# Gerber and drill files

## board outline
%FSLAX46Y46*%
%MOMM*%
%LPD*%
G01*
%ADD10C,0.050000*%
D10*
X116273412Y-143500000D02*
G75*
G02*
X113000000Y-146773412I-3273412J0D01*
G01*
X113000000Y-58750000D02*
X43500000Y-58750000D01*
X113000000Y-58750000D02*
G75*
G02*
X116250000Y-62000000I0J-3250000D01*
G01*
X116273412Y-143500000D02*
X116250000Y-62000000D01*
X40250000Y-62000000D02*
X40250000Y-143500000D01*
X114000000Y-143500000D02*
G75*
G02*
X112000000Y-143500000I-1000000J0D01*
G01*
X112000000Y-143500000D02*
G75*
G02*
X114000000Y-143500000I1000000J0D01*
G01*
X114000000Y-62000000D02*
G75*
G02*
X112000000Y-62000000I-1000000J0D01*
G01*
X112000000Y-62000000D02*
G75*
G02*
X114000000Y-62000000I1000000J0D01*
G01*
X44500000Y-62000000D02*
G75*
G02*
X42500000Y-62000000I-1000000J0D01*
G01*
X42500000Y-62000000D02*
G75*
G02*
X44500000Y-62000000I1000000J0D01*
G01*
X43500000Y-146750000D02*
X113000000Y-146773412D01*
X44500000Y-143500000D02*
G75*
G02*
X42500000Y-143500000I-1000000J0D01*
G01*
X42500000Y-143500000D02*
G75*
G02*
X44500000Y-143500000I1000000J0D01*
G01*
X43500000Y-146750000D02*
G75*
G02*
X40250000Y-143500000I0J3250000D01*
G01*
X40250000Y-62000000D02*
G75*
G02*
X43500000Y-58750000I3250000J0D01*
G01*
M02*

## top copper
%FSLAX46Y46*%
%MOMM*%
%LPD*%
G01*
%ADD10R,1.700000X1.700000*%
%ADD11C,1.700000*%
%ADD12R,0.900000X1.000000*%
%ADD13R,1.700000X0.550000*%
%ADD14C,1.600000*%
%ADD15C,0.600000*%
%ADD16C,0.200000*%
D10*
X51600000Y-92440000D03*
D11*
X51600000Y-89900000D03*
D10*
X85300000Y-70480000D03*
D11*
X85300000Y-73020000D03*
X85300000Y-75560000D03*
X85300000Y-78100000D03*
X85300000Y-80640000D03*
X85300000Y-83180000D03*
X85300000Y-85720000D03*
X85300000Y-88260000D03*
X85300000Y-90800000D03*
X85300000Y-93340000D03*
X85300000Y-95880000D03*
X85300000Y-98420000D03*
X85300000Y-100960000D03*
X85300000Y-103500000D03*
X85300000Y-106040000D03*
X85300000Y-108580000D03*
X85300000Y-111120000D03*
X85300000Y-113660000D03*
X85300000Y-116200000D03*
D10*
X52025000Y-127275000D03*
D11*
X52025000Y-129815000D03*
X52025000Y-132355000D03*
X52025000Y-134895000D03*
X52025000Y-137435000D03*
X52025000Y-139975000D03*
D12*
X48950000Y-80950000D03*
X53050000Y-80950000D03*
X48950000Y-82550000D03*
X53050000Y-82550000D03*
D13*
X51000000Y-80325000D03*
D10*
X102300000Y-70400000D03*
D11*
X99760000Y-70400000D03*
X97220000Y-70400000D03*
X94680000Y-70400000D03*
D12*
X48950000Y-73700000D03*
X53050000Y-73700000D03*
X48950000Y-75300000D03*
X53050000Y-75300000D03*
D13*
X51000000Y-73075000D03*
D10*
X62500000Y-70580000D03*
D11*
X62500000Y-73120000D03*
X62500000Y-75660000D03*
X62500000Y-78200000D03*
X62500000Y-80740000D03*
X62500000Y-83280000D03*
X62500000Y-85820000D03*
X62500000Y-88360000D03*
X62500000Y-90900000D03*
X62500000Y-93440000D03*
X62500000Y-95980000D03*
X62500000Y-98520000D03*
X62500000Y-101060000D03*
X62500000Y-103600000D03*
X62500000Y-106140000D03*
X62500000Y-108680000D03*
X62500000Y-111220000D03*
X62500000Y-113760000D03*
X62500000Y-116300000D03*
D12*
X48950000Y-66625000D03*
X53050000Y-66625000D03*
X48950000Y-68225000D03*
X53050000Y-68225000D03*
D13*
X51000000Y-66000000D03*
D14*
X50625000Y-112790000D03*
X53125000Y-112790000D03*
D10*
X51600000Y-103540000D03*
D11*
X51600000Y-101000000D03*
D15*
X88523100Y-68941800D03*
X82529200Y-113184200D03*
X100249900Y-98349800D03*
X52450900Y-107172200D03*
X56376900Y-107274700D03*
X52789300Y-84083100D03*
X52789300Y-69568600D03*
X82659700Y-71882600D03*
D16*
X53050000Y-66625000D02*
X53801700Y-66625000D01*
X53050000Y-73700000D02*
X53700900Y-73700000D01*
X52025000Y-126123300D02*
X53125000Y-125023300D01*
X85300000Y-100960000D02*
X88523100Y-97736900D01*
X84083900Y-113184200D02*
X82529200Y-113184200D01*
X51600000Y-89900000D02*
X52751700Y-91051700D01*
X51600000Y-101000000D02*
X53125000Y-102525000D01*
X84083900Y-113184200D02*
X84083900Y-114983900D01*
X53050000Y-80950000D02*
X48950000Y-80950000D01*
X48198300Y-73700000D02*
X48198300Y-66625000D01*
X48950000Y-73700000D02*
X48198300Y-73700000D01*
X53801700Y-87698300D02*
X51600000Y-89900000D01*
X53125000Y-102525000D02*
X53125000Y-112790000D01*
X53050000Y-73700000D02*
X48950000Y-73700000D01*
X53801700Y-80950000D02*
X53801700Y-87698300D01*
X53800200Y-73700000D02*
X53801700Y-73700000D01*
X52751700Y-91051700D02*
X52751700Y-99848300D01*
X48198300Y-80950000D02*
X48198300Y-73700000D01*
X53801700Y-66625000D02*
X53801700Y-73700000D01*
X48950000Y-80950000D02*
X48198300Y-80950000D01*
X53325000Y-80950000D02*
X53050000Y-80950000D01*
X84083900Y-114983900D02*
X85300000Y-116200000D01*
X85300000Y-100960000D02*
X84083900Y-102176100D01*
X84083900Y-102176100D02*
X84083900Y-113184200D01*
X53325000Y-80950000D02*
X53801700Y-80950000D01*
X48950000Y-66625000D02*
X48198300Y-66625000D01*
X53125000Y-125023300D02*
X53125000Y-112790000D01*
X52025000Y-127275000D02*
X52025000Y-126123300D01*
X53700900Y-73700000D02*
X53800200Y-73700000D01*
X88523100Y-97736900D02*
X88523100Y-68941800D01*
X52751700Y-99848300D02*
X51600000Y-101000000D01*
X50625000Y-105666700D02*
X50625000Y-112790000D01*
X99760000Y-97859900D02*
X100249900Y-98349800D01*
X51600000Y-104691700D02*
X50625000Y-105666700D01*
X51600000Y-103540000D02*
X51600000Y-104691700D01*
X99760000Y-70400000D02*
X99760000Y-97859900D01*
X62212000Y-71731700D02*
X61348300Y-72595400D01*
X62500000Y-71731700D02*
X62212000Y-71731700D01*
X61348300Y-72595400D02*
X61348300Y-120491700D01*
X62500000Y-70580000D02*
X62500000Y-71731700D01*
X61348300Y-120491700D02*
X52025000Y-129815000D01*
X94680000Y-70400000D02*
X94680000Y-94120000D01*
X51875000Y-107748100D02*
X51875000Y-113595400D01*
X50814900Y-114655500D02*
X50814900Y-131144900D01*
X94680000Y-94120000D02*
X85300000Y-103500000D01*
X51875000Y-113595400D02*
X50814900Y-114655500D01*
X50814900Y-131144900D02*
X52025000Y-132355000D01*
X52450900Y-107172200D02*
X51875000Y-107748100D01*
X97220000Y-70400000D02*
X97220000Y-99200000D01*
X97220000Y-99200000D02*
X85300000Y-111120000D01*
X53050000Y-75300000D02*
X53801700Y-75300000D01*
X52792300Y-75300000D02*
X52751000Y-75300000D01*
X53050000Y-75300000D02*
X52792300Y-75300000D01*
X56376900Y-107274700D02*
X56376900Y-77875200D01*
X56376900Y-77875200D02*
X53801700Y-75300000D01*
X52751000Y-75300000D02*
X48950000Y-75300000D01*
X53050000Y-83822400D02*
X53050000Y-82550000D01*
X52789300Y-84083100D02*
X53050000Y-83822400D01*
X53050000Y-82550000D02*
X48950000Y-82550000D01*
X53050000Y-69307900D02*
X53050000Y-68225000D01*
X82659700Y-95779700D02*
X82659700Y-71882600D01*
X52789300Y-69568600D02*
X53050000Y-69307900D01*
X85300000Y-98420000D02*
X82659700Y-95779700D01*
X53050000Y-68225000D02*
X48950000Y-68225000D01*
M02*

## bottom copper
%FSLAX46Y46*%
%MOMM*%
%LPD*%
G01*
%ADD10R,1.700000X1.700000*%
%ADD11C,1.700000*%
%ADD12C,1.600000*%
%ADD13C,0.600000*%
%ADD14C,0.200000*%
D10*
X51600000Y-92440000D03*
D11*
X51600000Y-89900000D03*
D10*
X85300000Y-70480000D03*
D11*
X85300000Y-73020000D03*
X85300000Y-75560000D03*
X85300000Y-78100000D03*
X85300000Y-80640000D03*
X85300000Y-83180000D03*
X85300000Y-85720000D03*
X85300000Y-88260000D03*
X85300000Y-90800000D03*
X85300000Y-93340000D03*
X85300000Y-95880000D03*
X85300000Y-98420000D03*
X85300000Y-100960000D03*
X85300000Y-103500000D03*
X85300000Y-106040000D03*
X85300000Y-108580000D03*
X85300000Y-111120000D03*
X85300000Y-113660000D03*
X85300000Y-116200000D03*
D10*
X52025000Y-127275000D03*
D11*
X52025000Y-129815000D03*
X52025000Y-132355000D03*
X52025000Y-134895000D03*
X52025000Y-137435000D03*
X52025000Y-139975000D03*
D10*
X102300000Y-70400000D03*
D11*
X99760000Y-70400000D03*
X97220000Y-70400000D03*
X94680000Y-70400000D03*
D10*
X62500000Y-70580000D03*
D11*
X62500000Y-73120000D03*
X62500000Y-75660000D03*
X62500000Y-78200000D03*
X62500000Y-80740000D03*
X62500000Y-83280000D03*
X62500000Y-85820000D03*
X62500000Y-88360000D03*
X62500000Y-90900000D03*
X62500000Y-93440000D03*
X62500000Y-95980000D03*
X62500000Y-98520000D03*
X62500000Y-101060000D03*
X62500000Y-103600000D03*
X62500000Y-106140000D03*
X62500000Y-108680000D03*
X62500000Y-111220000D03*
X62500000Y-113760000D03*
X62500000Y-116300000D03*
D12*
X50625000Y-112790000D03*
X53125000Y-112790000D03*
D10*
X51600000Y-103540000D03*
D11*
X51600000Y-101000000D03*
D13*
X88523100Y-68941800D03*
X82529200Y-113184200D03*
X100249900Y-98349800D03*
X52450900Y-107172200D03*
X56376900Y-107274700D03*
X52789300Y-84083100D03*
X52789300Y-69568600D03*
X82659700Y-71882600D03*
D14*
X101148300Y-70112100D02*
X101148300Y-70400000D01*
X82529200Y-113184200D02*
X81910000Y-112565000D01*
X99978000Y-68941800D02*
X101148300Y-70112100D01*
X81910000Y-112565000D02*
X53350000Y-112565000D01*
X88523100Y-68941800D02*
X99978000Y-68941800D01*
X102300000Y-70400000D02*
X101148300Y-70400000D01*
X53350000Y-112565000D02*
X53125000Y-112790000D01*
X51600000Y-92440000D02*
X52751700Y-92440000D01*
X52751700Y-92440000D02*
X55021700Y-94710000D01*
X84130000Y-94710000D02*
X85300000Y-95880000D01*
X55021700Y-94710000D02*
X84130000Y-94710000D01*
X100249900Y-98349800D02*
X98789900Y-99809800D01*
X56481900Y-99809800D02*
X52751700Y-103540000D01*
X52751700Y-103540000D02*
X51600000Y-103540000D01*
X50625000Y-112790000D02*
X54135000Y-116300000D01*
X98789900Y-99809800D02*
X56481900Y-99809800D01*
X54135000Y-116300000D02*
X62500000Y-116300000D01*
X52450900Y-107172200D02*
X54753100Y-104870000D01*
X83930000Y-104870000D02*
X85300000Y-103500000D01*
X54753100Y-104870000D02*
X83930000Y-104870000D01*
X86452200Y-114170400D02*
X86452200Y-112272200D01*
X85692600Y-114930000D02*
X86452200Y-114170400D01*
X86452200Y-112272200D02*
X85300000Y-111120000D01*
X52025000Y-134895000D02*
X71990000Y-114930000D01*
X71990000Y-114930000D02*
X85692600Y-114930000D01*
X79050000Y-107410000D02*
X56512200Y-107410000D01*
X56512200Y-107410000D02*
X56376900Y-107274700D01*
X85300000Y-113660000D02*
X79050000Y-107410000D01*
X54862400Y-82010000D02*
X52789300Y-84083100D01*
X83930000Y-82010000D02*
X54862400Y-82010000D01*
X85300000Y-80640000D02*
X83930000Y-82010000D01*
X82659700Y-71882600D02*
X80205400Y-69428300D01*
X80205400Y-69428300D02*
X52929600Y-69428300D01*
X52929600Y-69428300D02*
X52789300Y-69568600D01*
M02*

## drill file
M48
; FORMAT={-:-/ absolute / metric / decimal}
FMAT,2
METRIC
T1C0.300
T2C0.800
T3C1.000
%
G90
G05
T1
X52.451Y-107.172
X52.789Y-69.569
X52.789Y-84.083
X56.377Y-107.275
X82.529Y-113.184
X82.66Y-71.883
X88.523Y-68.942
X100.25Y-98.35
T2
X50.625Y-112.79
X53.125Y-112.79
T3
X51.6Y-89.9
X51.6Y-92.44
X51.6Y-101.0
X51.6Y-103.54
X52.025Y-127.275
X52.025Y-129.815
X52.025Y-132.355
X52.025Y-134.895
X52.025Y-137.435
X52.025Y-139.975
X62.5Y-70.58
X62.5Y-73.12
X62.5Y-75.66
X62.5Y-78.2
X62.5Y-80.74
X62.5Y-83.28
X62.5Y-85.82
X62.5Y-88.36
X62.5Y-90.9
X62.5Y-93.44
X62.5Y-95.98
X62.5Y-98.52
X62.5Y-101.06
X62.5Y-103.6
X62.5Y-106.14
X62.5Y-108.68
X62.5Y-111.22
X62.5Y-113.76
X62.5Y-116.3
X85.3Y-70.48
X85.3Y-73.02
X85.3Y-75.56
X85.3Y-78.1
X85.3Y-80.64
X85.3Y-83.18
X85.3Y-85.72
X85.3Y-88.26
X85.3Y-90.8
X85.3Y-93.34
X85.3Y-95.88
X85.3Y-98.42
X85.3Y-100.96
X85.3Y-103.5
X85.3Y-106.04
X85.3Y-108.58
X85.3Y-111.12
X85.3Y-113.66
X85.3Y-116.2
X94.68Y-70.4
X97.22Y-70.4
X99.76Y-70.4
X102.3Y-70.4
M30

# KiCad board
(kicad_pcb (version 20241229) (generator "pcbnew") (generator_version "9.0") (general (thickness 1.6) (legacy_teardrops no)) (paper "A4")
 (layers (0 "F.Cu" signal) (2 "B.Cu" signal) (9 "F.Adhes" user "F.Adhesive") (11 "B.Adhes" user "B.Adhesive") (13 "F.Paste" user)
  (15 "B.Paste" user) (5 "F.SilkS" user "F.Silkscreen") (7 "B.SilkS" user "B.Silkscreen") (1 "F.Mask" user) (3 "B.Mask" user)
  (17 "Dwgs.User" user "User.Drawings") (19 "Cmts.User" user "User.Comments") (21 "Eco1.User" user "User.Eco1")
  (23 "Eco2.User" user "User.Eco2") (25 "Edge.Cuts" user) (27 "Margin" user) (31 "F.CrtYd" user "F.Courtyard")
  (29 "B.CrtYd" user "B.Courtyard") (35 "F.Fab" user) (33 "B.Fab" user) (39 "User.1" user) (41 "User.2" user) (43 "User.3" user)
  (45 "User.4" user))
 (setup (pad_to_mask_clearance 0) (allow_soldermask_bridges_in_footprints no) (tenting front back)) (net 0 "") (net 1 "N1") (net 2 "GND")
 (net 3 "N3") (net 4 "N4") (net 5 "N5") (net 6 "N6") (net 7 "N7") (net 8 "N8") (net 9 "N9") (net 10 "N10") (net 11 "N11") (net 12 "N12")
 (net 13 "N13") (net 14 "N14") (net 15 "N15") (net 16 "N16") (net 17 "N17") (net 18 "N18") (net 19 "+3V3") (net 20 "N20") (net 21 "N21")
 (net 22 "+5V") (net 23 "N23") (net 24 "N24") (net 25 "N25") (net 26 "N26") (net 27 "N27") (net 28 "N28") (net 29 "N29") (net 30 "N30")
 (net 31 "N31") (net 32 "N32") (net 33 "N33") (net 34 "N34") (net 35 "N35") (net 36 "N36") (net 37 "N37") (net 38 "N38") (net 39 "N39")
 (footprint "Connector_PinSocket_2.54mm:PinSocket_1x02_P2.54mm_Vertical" (layer "F.Cu") (at 51.6 92.44 180)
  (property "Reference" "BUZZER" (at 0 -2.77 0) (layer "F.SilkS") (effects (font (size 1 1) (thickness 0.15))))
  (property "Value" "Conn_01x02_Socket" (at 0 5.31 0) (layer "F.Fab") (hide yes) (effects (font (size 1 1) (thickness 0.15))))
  (pad "1" thru_hole rect (at 0 0 180) (size 1.7 1.7) (drill 1) (layers "*.Cu" "*.Mask") (remove_unused_layers no) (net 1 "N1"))
  (pad "2" thru_hole circle (at 0 2.54 180) (size 1.7 1.7) (drill 1) (layers "*.Cu" "*.Mask") (remove_unused_layers no) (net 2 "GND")))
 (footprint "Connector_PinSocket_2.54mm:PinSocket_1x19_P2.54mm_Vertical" (layer "F.Cu") (at 85.3 70.48)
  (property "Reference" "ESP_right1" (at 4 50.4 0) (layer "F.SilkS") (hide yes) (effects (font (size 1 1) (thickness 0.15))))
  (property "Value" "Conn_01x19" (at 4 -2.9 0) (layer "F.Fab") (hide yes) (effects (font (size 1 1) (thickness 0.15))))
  (pad "1" thru_hole rect (at 0 0) (size 1.7 1.7) (drill 1) (layers "*.Cu" "*.Mask") (remove_unused_layers no) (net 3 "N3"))
  (pad "2" thru_hole circle (at 0 2.54) (size 1.7 1.7) (drill 1) (layers "*.Cu" "*.Mask") (remove_unused_layers no) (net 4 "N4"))
  (pad "3" thru_hole circle (at 0 5.08) (size 1.7 1.7) (drill 1) (layers "*.Cu" "*.Mask") (remove_unused_layers no) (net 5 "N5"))
  (pad "4" thru_hole circle (at 0 7.62) (size 1.7 1.7) (drill 1) (layers "*.Cu" "*.Mask") (remove_unused_layers no) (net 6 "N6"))
  (pad "5" thru_hole circle (at 0 10.16) (size 1.7 1.7) (drill 1) (layers "*.Cu" "*.Mask") (remove_unused_layers no) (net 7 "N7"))
  (pad "6" thru_hole circle (at 0 12.7) (size 1.7 1.7) (drill 1) (layers "*.Cu" "*.Mask") (remove_unused_layers no) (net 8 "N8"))
  (pad "7" thru_hole circle (at 0 15.24) (size 1.7 1.7) (drill 1) (layers "*.Cu" "*.Mask") (remove_unused_layers no) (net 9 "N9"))
  (pad "8" thru_hole circle (at 0 17.78) (size 1.7 1.7) (drill 1) (layers "*.Cu" "*.Mask") (remove_unused_layers no) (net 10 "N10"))
  (pad "9" thru_hole circle (at 0 20.32) (size 1.7 1.7) (drill 1) (layers "*.Cu" "*.Mask") (remove_unused_layers no) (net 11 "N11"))
  (pad "10" thru_hole circle (at 0 22.86) (size 1.7 1.7) (drill 1) (layers "*.Cu" "*.Mask") (remove_unused_layers no) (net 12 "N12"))
  (pad "11" thru_hole circle (at 0 25.4) (size 1.7 1.7) (drill 1) (layers "*.Cu" "*.Mask") (remove_unused_layers no) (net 1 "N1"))
  (pad "12" thru_hole circle (at 0 27.94) (size 1.7 1.7) (drill 1) (layers "*.Cu" "*.Mask") (remove_unused_layers no) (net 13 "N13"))
  (pad "13" thru_hole circle (at 0 30.48) (size 1.7 1.7) (drill 1) (layers "*.Cu" "*.Mask") (remove_unused_layers no) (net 2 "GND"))
  (pad "14" thru_hole circle (at 0 33.02) (size 1.7 1.7) (drill 1) (layers "*.Cu" "*.Mask") (remove_unused_layers no) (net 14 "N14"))
  (pad "15" thru_hole circle (at 0 35.56) (size 1.7 1.7) (drill 1) (layers "*.Cu" "*.Mask") (remove_unused_layers no) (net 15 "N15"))
  (pad "16" thru_hole circle (at 0 38.1) (size 1.7 1.7) (drill 1) (layers "*.Cu" "*.Mask") (remove_unused_layers no) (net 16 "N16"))
  (pad "17" thru_hole circle (at 0 40.64) (size 1.7 1.7) (drill 1) (layers "*.Cu" "*.Mask") (remove_unused_layers no) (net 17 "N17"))
  (pad "18" thru_hole circle (at 0 43.18) (size 1.7 1.7) (drill 1) (layers "*.Cu" "*.Mask") (remove_unused_layers no) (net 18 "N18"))
  (pad "19" thru_hole circle (at 0 45.72) (size 1.7 1.7) (drill 1) (layers "*.Cu" "*.Mask") (remove_unused_layers no) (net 2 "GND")))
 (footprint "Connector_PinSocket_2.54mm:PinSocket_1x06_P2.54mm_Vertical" (layer "F.Cu") (at 52.025 127.275)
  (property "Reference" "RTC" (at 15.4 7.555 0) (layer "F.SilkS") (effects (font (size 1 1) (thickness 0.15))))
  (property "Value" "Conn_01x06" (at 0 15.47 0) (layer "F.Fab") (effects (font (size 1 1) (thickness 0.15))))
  (pad "1" thru_hole rect (at 0 0) (size 1.7 1.7) (drill 1) (layers "*.Cu" "*.Mask") (remove_unused_layers no) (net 2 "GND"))
  (pad "2" thru_hole circle (at 0 2.54) (size 1.7 1.7) (drill 1) (layers "*.Cu" "*.Mask") (remove_unused_layers no) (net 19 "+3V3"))
  (pad "3" thru_hole circle (at 0 5.08) (size 1.7 1.7) (drill 1) (layers "*.Cu" "*.Mask") (remove_unused_layers no) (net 14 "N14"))
  (pad "4" thru_hole circle (at 0 7.62) (size 1.7 1.7) (drill 1) (layers "*.Cu" "*.Mask") (remove_unused_layers no) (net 17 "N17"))
  (pad "5" thru_hole circle (at 0 10.16) (size 1.7 1.7) (drill 1) (layers "*.Cu" "*.Mask") (remove_unused_layers no) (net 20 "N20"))
  (pad "6" thru_hole circle (at 0 12.7) (size 1.7 1.7) (drill 1) (layers "*.Cu" "*.Mask") (remove_unused_layers no) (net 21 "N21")))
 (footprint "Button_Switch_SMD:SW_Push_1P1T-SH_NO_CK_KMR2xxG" (layer "F.Cu") (at 51 81.75)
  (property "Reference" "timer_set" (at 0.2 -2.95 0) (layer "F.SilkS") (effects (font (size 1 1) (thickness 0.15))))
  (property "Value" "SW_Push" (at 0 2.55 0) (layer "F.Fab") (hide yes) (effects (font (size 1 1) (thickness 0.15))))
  (pad "1" smd rect (at -2.05 -0.8) (size 0.9 1) (layers "F.Cu" "F.Mask" "F.Paste") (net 2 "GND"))
  (pad "1" smd rect (at 2.05 -0.8) (size 0.9 1) (layers "F.Cu" "F.Mask" "F.Paste") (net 2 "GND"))
  (pad "2" smd rect (at -2.05 0.8) (size 0.9 1) (layers "F.Cu" "F.Mask" "F.Paste") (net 7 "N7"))
  (pad "2" smd rect (at 2.05 0.8) (size 0.9 1) (layers "F.Cu" "F.Mask" "F.Paste") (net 7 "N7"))
  (pad "SH" smd rect (at 0 -1.425) (size 1.7 0.55) (layers "F.Cu" "F.Mask" "F.Paste")))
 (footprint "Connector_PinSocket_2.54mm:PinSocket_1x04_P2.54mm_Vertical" (layer "F.Cu") (at 102.3 70.4 -90)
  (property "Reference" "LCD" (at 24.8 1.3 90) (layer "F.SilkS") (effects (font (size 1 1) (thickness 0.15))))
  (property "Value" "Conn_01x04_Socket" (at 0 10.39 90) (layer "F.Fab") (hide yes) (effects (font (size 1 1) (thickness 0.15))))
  (pad "1" thru_hole rect (at 0 0 270) (size 1.7 1.7) (drill 1) (layers "*.Cu" "*.Mask") (remove_unused_layers no) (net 2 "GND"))
  (pad "2" thru_hole circle (at 0 2.54 270) (size 1.7 1.7) (drill 1) (layers "*.Cu" "*.Mask") (remove_unused_layers no) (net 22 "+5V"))
  (pad "3" thru_hole circle (at 0 5.08 270) (size 1.7 1.7) (drill 1) (layers "*.Cu" "*.Mask") (remove_unused_layers no) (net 17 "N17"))
  (pad "4" thru_hole circle (at 0 7.62 270) (size 1.7 1.7) (drill 1) (layers "*.Cu" "*.Mask") (remove_unused_layers no) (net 14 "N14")))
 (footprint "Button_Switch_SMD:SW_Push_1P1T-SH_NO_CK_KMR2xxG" (layer "F.Cu") (at 51 74.5)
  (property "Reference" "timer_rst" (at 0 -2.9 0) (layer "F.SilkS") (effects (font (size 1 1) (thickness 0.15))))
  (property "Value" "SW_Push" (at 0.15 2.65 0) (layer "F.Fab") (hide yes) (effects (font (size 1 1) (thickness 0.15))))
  (pad "1" smd rect (at -2.05 -0.8) (size 0.9 1) (layers "F.Cu" "F.Mask" "F.Paste") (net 2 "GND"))
  (pad "1" smd rect (at 2.05 -0.8) (size 0.9 1) (layers "F.Cu" "F.Mask" "F.Paste") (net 2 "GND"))
  (pad "2" smd rect (at -2.05 0.8) (size 0.9 1) (layers "F.Cu" "F.Mask" "F.Paste") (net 18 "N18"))
  (pad "2" smd rect (at 2.05 0.8) (size 0.9 1) (layers "F.Cu" "F.Mask" "F.Paste") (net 18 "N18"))
  (pad "SH" smd rect (at 0 -1.425) (size 1.7 0.55) (layers "F.Cu" "F.Mask" "F.Paste")))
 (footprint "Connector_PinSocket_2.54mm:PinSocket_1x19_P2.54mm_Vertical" (layer "F.Cu") (at 62.5 70.58)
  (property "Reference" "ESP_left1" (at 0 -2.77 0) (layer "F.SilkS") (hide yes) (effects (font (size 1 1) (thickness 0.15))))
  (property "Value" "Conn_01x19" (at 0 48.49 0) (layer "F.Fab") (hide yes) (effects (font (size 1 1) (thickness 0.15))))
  (pad "1" thru_hole rect (at 0 0) (size 1.7 1.7) (drill 1) (layers "*.Cu" "*.Mask") (remove_unused_layers no) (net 19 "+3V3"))
  (pad "2" thru_hole circle (at 0 2.54) (size 1.7 1.7) (drill 1) (layers "*.Cu" "*.Mask") (remove_unused_layers no) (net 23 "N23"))
  (pad "3" thru_hole circle (at 0 5.08) (size 1.7 1.7) (drill 1) (layers "*.Cu" "*.Mask") (remove_unused_layers no) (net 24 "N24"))
  (pad "4" thru_hole circle (at 0 7.62) (size 1.7 1.7) (drill 1) (layers "*.Cu" "*.Mask") (remove_unused_layers no) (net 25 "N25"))
  (pad "5" thru_hole circle (at 0 10.16) (size 1.7 1.7) (drill 1) (layers "*.Cu" "*.Mask") (remove_unused_layers no) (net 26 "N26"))
  (pad "6" thru_hole circle (at 0 12.7) (size 1.7 1.7) (drill 1) (layers "*.Cu" "*.Mask") (remove_unused_layers no) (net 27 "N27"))
  (pad "7" thru_hole circle (at 0 15.24) (size 1.7 1.7) (drill 1) (layers "*.Cu" "*.Mask") (remove_unused_layers no) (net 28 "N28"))
  (pad "8" thru_hole circle (at 0 17.78) (size 1.7 1.7) (drill 1) (layers "*.Cu" "*.Mask") (remove_unused_layers no) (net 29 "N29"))
  (pad "9" thru_hole circle (at 0 20.32) (size 1.7 1.7) (drill 1) (layers "*.Cu" "*.Mask") (remove_unused_layers no) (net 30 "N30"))
  (pad "10" thru_hole circle (at 0 22.86) (size 1.7 1.7) (drill 1) (layers "*.Cu" "*.Mask") (remove_unused_layers no) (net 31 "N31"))
  (pad "11" thru_hole circle (at 0 25.4) (size 1.7 1.7) (drill 1) (layers "*.Cu" "*.Mask") (remove_unused_layers no) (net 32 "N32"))
  (pad "12" thru_hole circle (at 0 27.94) (size 1.7 1.7) (drill 1) (layers "*.Cu" "*.Mask") (remove_unused_layers no) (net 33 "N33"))
  (pad "13" thru_hole circle (at 0 30.48) (size 1.7 1.7) (drill 1) (layers "*.Cu" "*.Mask") (remove_unused_layers no) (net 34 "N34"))
  (pad "14" thru_hole circle (at 0 33.02) (size 1.7 1.7) (drill 1) (layers "*.Cu" "*.Mask") (remove_unused_layers no) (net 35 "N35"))
  (pad "15" thru_hole circle (at 0 35.56) (size 1.7 1.7) (drill 1) (layers "*.Cu" "*.Mask") (remove_unused_layers no) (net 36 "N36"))
  (pad "16" thru_hole circle (at 0 38.1) (size 1.7 1.7) (drill 1) (layers "*.Cu" "*.Mask") (remove_unused_layers no) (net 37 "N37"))
  (pad "17" thru_hole circle (at 0 40.64) (size 1.7 1.7) (drill 1) (layers "*.Cu" "*.Mask") (remove_unused_layers no) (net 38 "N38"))
  (pad "18" thru_hole circle (at 0 43.18) (size 1.7 1.7) (drill 1) (layers "*.Cu" "*.Mask") (remove_unused_layers no) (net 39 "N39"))
  (pad "19" thru_hole circle (at 0 45.72) (size 1.7 1.7) (drill 1) (layers "*.Cu" "*.Mask") (remove_unused_layers no) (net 22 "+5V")))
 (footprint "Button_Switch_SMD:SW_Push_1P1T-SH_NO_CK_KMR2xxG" (layer "F.Cu") (at 51 67.425)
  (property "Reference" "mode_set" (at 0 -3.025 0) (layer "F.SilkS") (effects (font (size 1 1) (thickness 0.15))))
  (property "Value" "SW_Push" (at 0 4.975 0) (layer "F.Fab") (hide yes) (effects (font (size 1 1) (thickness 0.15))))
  (pad "1" smd rect (at -2.05 -0.8) (size 0.9 1) (layers "F.Cu" "F.Mask" "F.Paste") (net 2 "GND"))
  (pad "1" smd rect (at 2.05 -0.8) (size 0.9 1) (layers "F.Cu" "F.Mask" "F.Paste") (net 2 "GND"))
  (pad "2" smd rect (at -2.05 0.8) (size 0.9 1) (layers "F.Cu" "F.Mask" "F.Paste") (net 13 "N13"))
  (pad "2" smd rect (at 2.05 0.8) (size 0.9 1) (layers "F.Cu" "F.Mask" "F.Paste") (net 13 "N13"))
  (pad "SH" smd rect (at 0 -1.425) (size 1.7 0.55) (layers "F.Cu" "F.Mask" "F.Paste")))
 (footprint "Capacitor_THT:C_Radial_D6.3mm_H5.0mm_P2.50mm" (layer "F.Cu") (at 50.625 112.79)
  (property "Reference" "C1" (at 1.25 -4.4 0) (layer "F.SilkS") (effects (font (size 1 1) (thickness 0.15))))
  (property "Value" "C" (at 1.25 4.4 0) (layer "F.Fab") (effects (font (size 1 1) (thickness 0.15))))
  (pad "1" thru_hole circle (at 0 0) (size 1.6 1.6) (drill 0.8) (layers "*.Cu" "*.Mask") (remove_unused_layers no) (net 22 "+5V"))
  (pad "2" thru_hole circle (at 2.5 0) (size 1.6 1.6) (drill 0.8) (layers "*.Cu" "*.Mask") (remove_unused_layers no) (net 2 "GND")))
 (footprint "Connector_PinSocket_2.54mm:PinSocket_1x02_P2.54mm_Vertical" (layer "F.Cu") (at 51.6 103.54 180)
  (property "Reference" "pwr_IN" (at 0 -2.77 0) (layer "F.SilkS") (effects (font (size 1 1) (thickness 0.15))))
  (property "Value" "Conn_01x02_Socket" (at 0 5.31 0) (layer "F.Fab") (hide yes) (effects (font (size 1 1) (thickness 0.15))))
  (pad "1" thru_hole rect (at 0 0 180) (size 1.7 1.7) (drill 1) (layers "*.Cu" "*.Mask") (remove_unused_layers no) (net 22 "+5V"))
  (pad "2" thru_hole circle (at 0 2.54 180) (size 1.7 1.7) (drill 1) (layers "*.Cu" "*.Mask") (remove_unused_layers no) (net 2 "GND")))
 (gr_arc (start 116.273412 143.5) (mid 115.314652 145.814652) (end 113 146.773412) (stroke (width 0.05) (type default)) (layer "Edge.Cuts"))
 (gr_line (start 113 58.75) (end 43.5 58.75) (stroke (width 0.05) (type default)) (layer "Edge.Cuts"))
 (gr_arc (start 113 58.75) (mid 115.298097 59.701903) (end 116.25 62) (stroke (width 0.05) (type default)) (layer "Edge.Cuts"))
 (gr_line (start 116.273412 143.5) (end 116.25 62) (stroke (width 0.05) (type default)) (layer "Edge.Cuts"))
 (gr_line (start 40.25 62) (end 40.25 143.5) (stroke (width 0.05) (type default)) (layer "Edge.Cuts"))
 (gr_circle (center 113 143.5) (end 114 143.5) (stroke (width 0.05) (type default)) (fill no) (layer "Edge.Cuts"))
 (gr_circle (center 113 62) (end 114 62) (stroke (width 0.05) (type default)) (fill no) (layer "Edge.Cuts"))
 (gr_circle (center 43.5 62) (end 42.5 62) (stroke (width 0.05) (type default)) (fill no) (layer "Edge.Cuts"))
 (gr_line (start 43.5 146.75) (end 113 146.773412) (stroke (width 0.05) (type default)) (layer "Edge.Cuts"))
 (gr_circle (center 43.5 143.5) (end 42.5 143.5) (stroke (width 0.05) (type default)) (fill no) (layer "Edge.Cuts"))
 (gr_arc (start 43.5 146.75) (mid 41.201903 145.798097) (end 40.25 143.5) (stroke (width 0.05) (type default)) (layer "Edge.Cuts"))
 (gr_arc (start 40.25 62) (mid 41.201903 59.701903) (end 43.5 58.75) (stroke (width 0.05) (type default)) (layer "Edge.Cuts"))
 (segment (start 53.05 66.625) (end 53.8017 66.625) (width 0.2) (layer "F.Cu") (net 2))
 (segment (start 53.05 73.7) (end 53.7009 73.7) (width 0.2) (layer "F.Cu") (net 2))
 (segment (start 52.025 126.1233) (end 53.125 125.0233) (width 0.2) (layer "F.Cu") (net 2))
 (segment (start 85.3 100.96) (end 88.5231 97.7369) (width 0.2) (layer "F.Cu") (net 2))
 (segment (start 84.0839 113.1842) (end 82.5292 113.1842) (width 0.2) (layer "F.Cu") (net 2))
 (segment (start 51.6 89.9) (end 52.7517 91.0517) (width 0.2) (layer "F.Cu") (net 2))
 (segment (start 51.6 101) (end 53.125 102.525) (width 0.2) (layer "F.Cu") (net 2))
 (segment (start 84.0839 113.1842) (end 84.0839 114.9839) (width 0.2) (layer "F.Cu") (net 2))
 (segment (start 53.05 80.95) (end 48.95 80.95) (width 0.2) (layer "F.Cu") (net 2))
 (segment (start 48.1983 73.7) (end 48.1983 66.625) (width 0.2) (layer "F.Cu") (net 2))
 (segment (start 48.95 73.7) (end 48.1983 73.7) (width 0.2) (layer "F.Cu") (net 2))
 (segment (start 53.8017 87.6983) (end 51.6 89.9) (width 0.2) (layer "F.Cu") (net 2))
 (segment (start 53.125 102.525) (end 53.125 112.79) (width 0.2) (layer "F.Cu") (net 2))
 (segment (start 53.05 73.7) (end 48.95 73.7) (width 0.2) (layer "F.Cu") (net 2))
 (segment (start 53.8017 80.95) (end 53.8017 87.6983) (width 0.2) (layer "F.Cu") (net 2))
 (segment (start 53.8002 73.7) (end 53.8017 73.7) (width 0.2) (layer "F.Cu") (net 2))
 (segment (start 52.7517 91.0517) (end 52.7517 99.8483) (width 0.2) (layer "F.Cu") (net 2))
 (segment (start 48.1983 80.95) (end 48.1983 73.7) (width 0.2) (layer "F.Cu") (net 2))
 (segment (start 53.8017 66.625) (end 53.8017 73.7) (width 0.2) (layer "F.Cu") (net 2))
 (segment (start 48.95 80.95) (end 48.1983 80.95) (width 0.2) (layer "F.Cu") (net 2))
 (segment (start 53.325 80.95) (end 53.05 80.95) (width 0.2) (layer "F.Cu") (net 2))
 (segment (start 84.0839 114.9839) (end 85.3 116.2) (width 0.2) (layer "F.Cu") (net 2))
 (segment (start 85.3 100.96) (end 84.0839 102.1761) (width 0.2) (layer "F.Cu") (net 2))
 (segment (start 84.0839 102.1761) (end 84.0839 113.1842) (width 0.2) (layer "F.Cu") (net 2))
 (segment (start 53.325 80.95) (end 53.8017 80.95) (width 0.2) (layer "F.Cu") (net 2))
 (segment (start 48.95 66.625) (end 48.1983 66.625) (width 0.2) (layer "F.Cu") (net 2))
 (segment (start 53.125 125.0233) (end 53.125 112.79) (width 0.2) (layer "F.Cu") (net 2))
 (segment (start 52.025 127.275) (end 52.025 126.1233) (width 0.2) (layer "F.Cu") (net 2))
 (segment (start 53.7009 73.7) (end 53.8002 73.7) (width 0.2) (layer "F.Cu") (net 2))
 (segment (start 88.5231 97.7369) (end 88.5231 68.9418) (width 0.2) (layer "F.Cu") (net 2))
 (segment (start 52.7517 99.8483) (end 51.6 101) (width 0.2) (layer "F.Cu") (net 2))
 (via (at 88.5231 68.9418) (size 0.6) (drill 0.3) (layers "F.Cu" "B.Cu") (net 2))
 (via (at 82.5292 113.1842) (size 0.6) (drill 0.3) (layers "F.Cu" "B.Cu") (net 2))
 (segment (start 101.1483 70.1121) (end 101.1483 70.4) (width 0.2) (layer "B.Cu") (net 2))
 (segment (start 82.5292 113.1842) (end 81.91 112.565) (width 0.2) (layer "B.Cu") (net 2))
 (segment (start 99.978 68.9418) (end 101.1483 70.1121) (width 0.2) (layer "B.Cu") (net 2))
 (segment (start 81.91 112.565) (end 53.35 112.565) (width 0.2) (layer "B.Cu") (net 2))
 (segment (start 88.5231 68.9418) (end 99.978 68.9418) (width 0.2) (layer "B.Cu") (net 2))
 (segment (start 102.3 70.4) (end 101.1483 70.4) (width 0.2) (layer "B.Cu") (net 2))
 (segment (start 53.35 112.565) (end 53.125 112.79) (width 0.2) (layer "B.Cu") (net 2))
 (segment (start 51.6 92.44) (end 52.7517 92.44) (width 0.2) (layer "B.Cu") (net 1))
 (segment (start 52.7517 92.44) (end 55.0217 94.71) (width 0.2) (layer "B.Cu") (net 1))
 (segment (start 84.13 94.71) (end 85.3 95.88) (width 0.2) (layer "B.Cu") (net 1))
 (segment (start 55.0217 94.71) (end 84.13 94.71) (width 0.2) (layer "B.Cu") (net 1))
 (segment (start 50.625 105.6667) (end 50.625 112.79) (width 0.2) (layer "F.Cu") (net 22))
 (segment (start 99.76 97.8599) (end 100.2499 98.3498) (width 0.2) (layer "F.Cu") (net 22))
 (segment (start 51.6 104.6917) (end 50.625 105.6667) (width 0.2) (layer "F.Cu") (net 22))
 (segment (start 51.6 103.54) (end 51.6 104.6917) (width 0.2) (layer "F.Cu") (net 22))
 (segment (start 99.76 70.4) (end 99.76 97.8599) (width 0.2) (layer "F.Cu") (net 22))
 (via (at 100.2499 98.3498) (size 0.6) (drill 0.3) (layers "F.Cu" "B.Cu") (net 22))
 (segment (start 100.2499 98.3498) (end 98.7899 99.8098) (width 0.2) (layer "B.Cu") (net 22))
 (segment (start 56.4819 99.8098) (end 52.7517 103.54) (width 0.2) (layer "B.Cu") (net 22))
 (segment (start 52.7517 103.54) (end 51.6 103.54) (width 0.2) (layer "B.Cu") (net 22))
 (segment (start 50.625 112.79) (end 54.135 116.3) (width 0.2) (layer "B.Cu") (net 22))
 (segment (start 98.7899 99.8098) (end 56.4819 99.8098) (width 0.2) (layer "B.Cu") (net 22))
 (segment (start 54.135 116.3) (end 62.5 116.3) (width 0.2) (layer "B.Cu") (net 22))
 (segment (start 62.212 71.7317) (end 61.3483 72.5954) (width 0.2) (layer "F.Cu") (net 19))
 (segment (start 62.5 71.7317) (end 62.212 71.7317) (width 0.2) (layer "F.Cu") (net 19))
 (segment (start 61.3483 72.5954) (end 61.3483 120.4917) (width 0.2) (layer "F.Cu") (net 19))
 (segment (start 62.5 70.58) (end 62.5 71.7317) (width 0.2) (layer "F.Cu") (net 19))
 (segment (start 61.3483 120.4917) (end 52.025 129.815) (width 0.2) (layer "F.Cu") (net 19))
 (segment (start 94.68 70.4) (end 94.68 94.12) (width 0.2) (layer "F.Cu") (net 14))
 (segment (start 51.875 107.7481) (end 51.875 113.5954) (width 0.2) (layer "F.Cu") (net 14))
 (segment (start 50.8149 114.6555) (end 50.8149 131.1449) (width 0.2) (layer "F.Cu") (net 14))
 (segment (start 94.68 94.12) (end 85.3 103.5) (width 0.2) (layer "F.Cu") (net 14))
 (segment (start 51.875 113.5954) (end 50.8149 114.6555) (width 0.2) (layer "F.Cu") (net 14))
 (segment (start 50.8149 131.1449) (end 52.025 132.355) (width 0.2) (layer "F.Cu") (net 14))
 (segment (start 52.4509 107.1722) (end 51.875 107.7481) (width 0.2) (layer "F.Cu") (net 14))
 (via (at 52.4509 107.1722) (size 0.6) (drill 0.3) (layers "F.Cu" "B.Cu") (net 14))
 (segment (start 52.4509 107.1722) (end 54.7531 104.87) (width 0.2) (layer "B.Cu") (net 14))
 (segment (start 83.93 104.87) (end 85.3 103.5) (width 0.2) (layer "B.Cu") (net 14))
 (segment (start 54.7531 104.87) (end 83.93 104.87) (width 0.2) (layer "B.Cu") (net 14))
 (segment (start 97.22 70.4) (end 97.22 99.2) (width 0.2) (layer "F.Cu") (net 17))
 (segment (start 97.22 99.2) (end 85.3 111.12) (width 0.2) (layer "F.Cu") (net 17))
 (segment (start 86.4522 114.1704) (end 86.4522 112.2722) (width 0.2) (layer "B.Cu") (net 17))
 (segment (start 85.6926 114.93) (end 86.4522 114.1704) (width 0.2) (layer "B.Cu") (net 17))
 (segment (start 86.4522 112.2722) (end 85.3 111.12) (width 0.2) (layer "B.Cu") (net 17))
 (segment (start 52.025 134.895) (end 71.99 114.93) (width 0.2) (layer "B.Cu") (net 17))
 (segment (start 71.99 114.93) (end 85.6926 114.93) (width 0.2) (layer "B.Cu") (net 17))
 (segment (start 53.05 75.3) (end 53.8017 75.3) (width 0.2) (layer "F.Cu") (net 18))
 (segment (start 52.7923 75.3) (end 52.751 75.3) (width 0.2) (layer "F.Cu") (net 18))
 (segment (start 53.05 75.3) (end 52.7923 75.3) (width 0.2) (layer "F.Cu") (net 18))
 (segment (start 56.3769 107.2747) (end 56.3769 77.8752) (width 0.2) (layer "F.Cu") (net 18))
 (segment (start 56.3769 77.8752) (end 53.8017 75.3) (width 0.2) (layer "F.Cu") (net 18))
 (segment (start 52.751 75.3) (end 48.95 75.3) (width 0.2) (layer "F.Cu") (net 18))
 (via (at 56.3769 107.2747) (size 0.6) (drill 0.3) (layers "F.Cu" "B.Cu") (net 18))
 (segment (start 79.05 107.41) (end 56.5122 107.41) (width 0.2) (layer "B.Cu") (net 18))
 (segment (start 56.5122 107.41) (end 56.3769 107.2747) (width 0.2) (layer "B.Cu") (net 18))
 (segment (start 85.3 113.66) (end 79.05 107.41) (width 0.2) (layer "B.Cu") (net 18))
 (segment (start 53.05 83.8224) (end 53.05 82.55) (width 0.2) (layer "F.Cu") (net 7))
 (segment (start 52.7893 84.0831) (end 53.05 83.8224) (width 0.2) (layer "F.Cu") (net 7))
 (segment (start 53.05 82.55) (end 48.95 82.55) (width 0.2) (layer "F.Cu") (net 7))
 (via (at 52.7893 84.0831) (size 0.6) (drill 0.3) (layers "F.Cu" "B.Cu") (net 7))
 (segment (start 54.8624 82.01) (end 52.7893 84.0831) (width 0.2) (layer "B.Cu") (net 7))
 (segment (start 83.93 82.01) (end 54.8624 82.01) (width 0.2) (layer "B.Cu") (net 7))
 (segment (start 85.3 80.64) (end 83.93 82.01) (width 0.2) (layer "B.Cu") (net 7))
 (segment (start 53.05 69.3079) (end 53.05 68.225) (width 0.2) (layer "F.Cu") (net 13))
 (segment (start 82.6597 95.7797) (end 82.6597 71.8826) (width 0.2) (layer "F.Cu") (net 13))
 (segment (start 52.7893 69.5686) (end 53.05 69.3079) (width 0.2) (layer "F.Cu") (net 13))
 (segment (start 85.3 98.42) (end 82.6597 95.7797) (width 0.2) (layer "F.Cu") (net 13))
 (segment (start 53.05 68.225) (end 48.95 68.225) (width 0.2) (layer "F.Cu") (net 13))
 (via (at 52.7893 69.5686) (size 0.6) (drill 0.3) (layers "F.Cu" "B.Cu") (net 13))
 (via (at 82.6597 71.8826) (size 0.6) (drill 0.3) (layers "F.Cu" "B.Cu") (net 13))
 (segment (start 82.6597 71.8826) (end 80.2054 69.4283) (width 0.2) (layer "B.Cu") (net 13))
 (segment (start 80.2054 69.4283) (end 52.9296 69.4283) (width 0.2) (layer "B.Cu") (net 13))
 (segment (start 52.9296 69.4283) (end 52.7893 69.5686) (width 0.2) (layer "B.Cu") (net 13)))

